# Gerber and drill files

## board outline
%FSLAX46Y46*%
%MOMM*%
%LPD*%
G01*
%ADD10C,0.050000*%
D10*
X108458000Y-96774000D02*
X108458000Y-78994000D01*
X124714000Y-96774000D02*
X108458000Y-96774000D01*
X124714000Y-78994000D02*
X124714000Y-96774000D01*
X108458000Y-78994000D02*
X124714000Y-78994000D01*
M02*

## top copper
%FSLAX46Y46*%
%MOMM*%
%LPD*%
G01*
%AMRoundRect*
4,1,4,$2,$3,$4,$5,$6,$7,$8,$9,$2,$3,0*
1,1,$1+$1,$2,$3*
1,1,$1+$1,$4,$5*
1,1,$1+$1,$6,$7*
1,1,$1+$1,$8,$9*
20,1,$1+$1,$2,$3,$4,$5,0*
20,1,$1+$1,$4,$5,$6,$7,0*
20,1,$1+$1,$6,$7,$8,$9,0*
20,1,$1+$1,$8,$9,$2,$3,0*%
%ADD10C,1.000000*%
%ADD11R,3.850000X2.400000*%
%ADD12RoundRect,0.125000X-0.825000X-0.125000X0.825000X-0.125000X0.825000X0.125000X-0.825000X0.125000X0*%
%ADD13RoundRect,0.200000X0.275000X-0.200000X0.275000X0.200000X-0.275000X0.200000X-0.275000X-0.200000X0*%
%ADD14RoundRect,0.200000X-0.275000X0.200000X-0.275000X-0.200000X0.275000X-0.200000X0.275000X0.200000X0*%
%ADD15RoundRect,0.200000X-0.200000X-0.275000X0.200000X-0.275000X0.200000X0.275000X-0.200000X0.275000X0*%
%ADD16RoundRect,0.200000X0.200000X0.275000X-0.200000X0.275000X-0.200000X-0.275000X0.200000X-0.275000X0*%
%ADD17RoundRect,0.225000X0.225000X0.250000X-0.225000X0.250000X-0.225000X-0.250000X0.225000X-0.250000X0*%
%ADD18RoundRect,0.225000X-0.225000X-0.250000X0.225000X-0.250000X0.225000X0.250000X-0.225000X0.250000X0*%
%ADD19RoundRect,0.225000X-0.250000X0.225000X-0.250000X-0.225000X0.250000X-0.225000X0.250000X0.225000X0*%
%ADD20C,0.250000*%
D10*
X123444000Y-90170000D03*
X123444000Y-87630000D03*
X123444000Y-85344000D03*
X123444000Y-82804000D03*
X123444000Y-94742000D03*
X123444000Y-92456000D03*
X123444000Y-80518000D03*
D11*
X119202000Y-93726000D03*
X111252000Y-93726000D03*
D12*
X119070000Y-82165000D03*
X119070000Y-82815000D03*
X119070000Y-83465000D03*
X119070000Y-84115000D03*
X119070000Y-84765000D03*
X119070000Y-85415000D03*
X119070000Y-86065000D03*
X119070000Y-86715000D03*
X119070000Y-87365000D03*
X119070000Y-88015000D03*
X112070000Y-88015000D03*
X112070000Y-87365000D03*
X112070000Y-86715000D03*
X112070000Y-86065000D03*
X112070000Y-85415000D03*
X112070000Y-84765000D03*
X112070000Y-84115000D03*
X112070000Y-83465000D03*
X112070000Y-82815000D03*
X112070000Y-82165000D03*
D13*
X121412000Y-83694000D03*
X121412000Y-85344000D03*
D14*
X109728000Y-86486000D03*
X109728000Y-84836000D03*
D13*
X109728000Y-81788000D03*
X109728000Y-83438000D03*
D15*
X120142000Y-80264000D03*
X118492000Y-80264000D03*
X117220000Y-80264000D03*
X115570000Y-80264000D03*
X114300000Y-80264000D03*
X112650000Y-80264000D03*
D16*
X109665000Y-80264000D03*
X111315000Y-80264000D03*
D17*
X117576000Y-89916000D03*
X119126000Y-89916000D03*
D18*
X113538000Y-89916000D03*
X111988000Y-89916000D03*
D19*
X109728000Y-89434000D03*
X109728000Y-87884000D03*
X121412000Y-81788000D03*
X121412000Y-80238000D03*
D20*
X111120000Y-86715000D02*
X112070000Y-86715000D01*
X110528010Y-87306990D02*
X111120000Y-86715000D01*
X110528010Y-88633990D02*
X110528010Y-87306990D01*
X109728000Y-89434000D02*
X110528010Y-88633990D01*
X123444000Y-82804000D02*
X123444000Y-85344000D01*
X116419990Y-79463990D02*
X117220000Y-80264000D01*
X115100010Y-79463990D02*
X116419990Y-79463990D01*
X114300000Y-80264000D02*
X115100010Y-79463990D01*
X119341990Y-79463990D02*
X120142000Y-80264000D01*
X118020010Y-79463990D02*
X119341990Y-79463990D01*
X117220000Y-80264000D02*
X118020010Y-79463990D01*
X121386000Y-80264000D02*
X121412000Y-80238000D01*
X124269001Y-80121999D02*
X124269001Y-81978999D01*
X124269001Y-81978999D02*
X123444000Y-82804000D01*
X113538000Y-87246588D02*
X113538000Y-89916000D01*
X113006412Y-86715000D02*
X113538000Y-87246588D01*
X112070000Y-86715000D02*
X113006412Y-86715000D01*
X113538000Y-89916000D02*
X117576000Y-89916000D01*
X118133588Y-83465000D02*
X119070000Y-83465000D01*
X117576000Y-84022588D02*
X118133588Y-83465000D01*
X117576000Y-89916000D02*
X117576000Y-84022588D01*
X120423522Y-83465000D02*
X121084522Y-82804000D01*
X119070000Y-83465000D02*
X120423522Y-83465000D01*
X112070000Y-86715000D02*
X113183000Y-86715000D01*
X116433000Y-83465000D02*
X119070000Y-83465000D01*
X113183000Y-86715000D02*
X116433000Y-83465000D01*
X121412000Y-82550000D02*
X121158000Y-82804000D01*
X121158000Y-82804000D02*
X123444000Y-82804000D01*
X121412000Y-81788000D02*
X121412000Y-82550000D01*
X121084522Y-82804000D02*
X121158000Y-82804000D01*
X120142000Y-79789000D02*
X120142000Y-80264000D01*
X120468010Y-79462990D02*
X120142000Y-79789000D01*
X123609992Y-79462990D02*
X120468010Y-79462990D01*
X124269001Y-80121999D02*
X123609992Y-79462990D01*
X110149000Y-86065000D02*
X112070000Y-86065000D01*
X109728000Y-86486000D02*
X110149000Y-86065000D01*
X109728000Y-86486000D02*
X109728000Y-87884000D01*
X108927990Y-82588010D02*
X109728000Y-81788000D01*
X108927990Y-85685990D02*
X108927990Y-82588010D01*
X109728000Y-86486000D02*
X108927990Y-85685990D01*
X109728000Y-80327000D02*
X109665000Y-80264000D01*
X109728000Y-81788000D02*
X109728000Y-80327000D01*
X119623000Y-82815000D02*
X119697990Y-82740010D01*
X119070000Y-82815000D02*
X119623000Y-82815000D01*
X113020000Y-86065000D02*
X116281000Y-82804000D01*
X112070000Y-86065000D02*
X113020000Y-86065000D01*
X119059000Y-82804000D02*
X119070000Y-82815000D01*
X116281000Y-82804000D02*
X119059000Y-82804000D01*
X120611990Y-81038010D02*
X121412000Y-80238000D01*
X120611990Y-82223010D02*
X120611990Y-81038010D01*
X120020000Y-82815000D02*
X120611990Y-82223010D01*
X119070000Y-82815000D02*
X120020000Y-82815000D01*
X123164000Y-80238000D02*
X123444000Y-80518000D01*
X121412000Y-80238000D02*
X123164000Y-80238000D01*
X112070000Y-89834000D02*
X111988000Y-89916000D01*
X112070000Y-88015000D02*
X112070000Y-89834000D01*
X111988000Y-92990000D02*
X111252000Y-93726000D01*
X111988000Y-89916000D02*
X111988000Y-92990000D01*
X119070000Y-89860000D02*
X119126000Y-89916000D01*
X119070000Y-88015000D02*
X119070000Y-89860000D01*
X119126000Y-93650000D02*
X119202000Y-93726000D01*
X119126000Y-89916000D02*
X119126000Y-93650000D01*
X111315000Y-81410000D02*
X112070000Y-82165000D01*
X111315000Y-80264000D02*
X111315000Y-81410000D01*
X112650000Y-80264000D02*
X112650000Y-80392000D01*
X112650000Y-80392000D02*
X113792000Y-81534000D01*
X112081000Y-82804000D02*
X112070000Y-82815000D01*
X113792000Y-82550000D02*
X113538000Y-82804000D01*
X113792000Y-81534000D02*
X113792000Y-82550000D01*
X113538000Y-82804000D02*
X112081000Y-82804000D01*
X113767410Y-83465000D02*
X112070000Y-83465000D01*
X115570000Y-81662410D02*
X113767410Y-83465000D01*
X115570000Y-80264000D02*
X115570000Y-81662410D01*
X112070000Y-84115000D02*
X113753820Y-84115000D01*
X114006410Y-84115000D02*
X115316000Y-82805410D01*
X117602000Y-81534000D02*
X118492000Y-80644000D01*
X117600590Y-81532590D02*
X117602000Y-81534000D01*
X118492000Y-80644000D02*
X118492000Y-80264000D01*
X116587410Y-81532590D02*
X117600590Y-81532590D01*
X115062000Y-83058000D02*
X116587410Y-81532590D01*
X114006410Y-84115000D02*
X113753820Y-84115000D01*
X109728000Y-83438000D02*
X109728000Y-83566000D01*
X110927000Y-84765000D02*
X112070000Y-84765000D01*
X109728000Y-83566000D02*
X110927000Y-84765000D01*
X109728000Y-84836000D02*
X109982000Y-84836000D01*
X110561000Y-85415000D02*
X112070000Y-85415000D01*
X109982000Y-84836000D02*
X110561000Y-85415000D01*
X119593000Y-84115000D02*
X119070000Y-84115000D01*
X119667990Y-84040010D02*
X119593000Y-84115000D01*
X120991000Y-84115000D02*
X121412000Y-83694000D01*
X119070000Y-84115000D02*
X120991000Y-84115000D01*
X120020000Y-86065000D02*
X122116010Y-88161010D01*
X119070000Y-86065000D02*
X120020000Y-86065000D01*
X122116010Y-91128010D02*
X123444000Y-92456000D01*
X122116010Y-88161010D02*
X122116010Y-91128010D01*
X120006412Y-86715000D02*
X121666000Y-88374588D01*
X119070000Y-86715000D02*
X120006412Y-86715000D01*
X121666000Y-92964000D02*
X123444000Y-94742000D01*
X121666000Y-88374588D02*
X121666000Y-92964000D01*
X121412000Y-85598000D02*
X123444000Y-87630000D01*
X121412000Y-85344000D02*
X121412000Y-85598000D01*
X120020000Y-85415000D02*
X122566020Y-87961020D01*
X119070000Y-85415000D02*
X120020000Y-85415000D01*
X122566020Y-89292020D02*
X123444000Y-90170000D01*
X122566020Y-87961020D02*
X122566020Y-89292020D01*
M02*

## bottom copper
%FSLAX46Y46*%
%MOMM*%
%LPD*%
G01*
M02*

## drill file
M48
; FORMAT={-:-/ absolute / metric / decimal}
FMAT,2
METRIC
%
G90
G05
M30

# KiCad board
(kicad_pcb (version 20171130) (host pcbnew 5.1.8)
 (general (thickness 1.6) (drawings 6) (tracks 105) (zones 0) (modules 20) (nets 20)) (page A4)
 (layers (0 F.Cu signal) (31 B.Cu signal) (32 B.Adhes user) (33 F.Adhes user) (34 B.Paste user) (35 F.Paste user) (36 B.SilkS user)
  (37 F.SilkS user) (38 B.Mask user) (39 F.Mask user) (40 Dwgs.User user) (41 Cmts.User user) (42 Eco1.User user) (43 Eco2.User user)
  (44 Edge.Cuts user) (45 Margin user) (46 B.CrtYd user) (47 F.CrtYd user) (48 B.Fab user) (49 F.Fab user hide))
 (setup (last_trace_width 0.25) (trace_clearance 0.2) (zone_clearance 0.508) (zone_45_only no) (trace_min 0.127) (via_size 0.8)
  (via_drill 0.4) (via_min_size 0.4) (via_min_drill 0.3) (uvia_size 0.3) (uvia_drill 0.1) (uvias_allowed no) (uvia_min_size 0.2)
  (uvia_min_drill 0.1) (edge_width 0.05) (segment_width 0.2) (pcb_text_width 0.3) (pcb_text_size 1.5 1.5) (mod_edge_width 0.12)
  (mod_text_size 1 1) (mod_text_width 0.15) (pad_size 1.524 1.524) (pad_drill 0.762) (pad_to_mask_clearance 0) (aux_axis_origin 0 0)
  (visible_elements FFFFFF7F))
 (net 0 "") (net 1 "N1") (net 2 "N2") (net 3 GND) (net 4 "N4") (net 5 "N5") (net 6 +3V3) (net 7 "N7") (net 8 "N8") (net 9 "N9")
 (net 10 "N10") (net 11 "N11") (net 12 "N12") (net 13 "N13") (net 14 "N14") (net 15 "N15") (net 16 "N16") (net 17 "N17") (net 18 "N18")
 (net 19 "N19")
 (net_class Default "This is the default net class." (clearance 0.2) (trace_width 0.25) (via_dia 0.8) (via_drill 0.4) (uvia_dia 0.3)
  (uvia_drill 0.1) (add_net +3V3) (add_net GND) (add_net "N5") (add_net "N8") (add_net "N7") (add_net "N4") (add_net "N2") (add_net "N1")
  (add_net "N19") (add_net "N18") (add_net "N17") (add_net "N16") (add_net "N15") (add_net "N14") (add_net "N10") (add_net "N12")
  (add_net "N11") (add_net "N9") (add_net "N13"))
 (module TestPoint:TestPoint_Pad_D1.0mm (layer F.Cu) (at 123.444 90.17)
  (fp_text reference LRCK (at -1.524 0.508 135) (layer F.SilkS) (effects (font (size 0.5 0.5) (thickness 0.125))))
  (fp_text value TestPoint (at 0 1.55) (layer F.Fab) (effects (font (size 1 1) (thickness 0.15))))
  (pad 1 smd circle (at 0 0) (size 1 1) (layers F.Cu F.Mask) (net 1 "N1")))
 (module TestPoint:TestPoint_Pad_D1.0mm (layer F.Cu) (at 123.444 87.63)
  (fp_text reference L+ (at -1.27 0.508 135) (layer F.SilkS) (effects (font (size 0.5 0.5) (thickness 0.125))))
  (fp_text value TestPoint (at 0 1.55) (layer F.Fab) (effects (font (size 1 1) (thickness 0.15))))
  (pad 1 smd circle (at 0 0) (size 1 1) (layers F.Cu F.Mask) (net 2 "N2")))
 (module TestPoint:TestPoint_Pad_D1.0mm (layer F.Cu) (at 123.444 85.344)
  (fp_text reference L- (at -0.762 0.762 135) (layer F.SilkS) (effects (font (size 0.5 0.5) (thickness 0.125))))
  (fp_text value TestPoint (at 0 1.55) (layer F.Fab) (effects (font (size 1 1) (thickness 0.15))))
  (pad 1 smd circle (at 0 0) (size 1 1) (layers F.Cu F.Mask) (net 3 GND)))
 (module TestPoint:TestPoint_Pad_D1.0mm (layer F.Cu) (at 123.444 82.804)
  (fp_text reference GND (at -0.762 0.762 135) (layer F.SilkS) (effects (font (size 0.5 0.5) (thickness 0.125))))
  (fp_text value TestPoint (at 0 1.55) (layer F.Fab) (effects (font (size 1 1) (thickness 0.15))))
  (pad 1 smd circle (at 0 0) (size 1 1) (layers F.Cu F.Mask) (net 3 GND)))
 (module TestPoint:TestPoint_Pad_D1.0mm (layer F.Cu) (at 123.444 94.742)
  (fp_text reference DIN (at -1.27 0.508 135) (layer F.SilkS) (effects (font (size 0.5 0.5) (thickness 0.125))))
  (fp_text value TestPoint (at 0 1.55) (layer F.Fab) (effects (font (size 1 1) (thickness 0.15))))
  (pad 1 smd circle (at 0 0) (size 1 1) (layers F.Cu F.Mask) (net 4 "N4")))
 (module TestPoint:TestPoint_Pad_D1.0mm (layer F.Cu) (at 123.444 92.456)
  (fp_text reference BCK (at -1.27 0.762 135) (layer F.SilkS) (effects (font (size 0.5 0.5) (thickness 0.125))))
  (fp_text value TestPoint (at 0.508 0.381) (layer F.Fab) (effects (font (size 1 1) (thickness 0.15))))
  (pad 1 smd circle (at 0 0) (size 1 1) (layers F.Cu F.Mask) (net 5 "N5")))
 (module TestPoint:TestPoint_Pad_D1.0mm (layer F.Cu) (at 123.444 80.518)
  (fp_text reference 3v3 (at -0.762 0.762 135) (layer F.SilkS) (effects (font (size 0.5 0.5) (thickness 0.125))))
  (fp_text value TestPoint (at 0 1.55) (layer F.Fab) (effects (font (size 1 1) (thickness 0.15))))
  (pad 1 smd circle (at 0 0) (size 1 1) (layers F.Cu F.Mask) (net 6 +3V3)))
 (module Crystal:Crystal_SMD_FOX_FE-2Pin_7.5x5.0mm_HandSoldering (layer F.Cu) (at 115.227 93.726)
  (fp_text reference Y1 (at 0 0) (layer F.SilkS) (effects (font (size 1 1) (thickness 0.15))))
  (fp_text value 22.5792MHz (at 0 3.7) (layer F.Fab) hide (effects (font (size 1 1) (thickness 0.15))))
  (pad 2 smd rect (at 3.975 0) (size 3.85 2.4) (layers F.Cu F.Paste F.Mask) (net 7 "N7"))
  (pad 1 smd rect (at -3.975 0) (size 3.85 2.4) (layers F.Cu F.Paste F.Mask) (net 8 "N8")))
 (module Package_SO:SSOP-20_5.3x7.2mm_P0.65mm (layer F.Cu) (at 115.57 85.09)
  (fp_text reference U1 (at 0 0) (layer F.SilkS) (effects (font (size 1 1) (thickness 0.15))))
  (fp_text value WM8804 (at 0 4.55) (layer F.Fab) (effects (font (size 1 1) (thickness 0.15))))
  (pad 20 smd roundrect (at 3.5 -2.925) (size 1.9 0.5) (layers F.Cu F.Paste F.Mask) (roundrect_rratio 0.25) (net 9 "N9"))
  (pad 19 smd roundrect (at 3.5 -2.275) (size 1.9 0.5) (layers F.Cu F.Paste F.Mask) (roundrect_rratio 0.25) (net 6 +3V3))
  (pad 18 smd roundrect (at 3.5 -1.625) (size 1.9 0.5) (layers F.Cu F.Paste F.Mask) (roundrect_rratio 0.25) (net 3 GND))
  (pad 17 smd roundrect (at 3.5 -0.975) (size 1.9 0.5) (layers F.Cu F.Paste F.Mask) (roundrect_rratio 0.25) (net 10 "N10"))
  (pad 16 smd roundrect (at 3.5 -0.325) (size 1.9 0.5) (layers F.Cu F.Paste F.Mask) (roundrect_rratio 0.25) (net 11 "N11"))
  (pad 15 smd roundrect (at 3.5 0.325) (size 1.9 0.5) (layers F.Cu F.Paste F.Mask) (roundrect_rratio 0.25) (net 1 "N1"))
  (pad 14 smd roundrect (at 3.5 0.975) (size 1.9 0.5) (layers F.Cu F.Paste F.Mask) (roundrect_rratio 0.25) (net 5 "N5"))
  (pad 13 smd roundrect (at 3.5 1.625) (size 1.9 0.5) (layers F.Cu F.Paste F.Mask) (roundrect_rratio 0.25) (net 4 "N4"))
  (pad 12 smd roundrect (at 3.5 2.275) (size 1.9 0.5) (layers F.Cu F.Paste F.Mask) (roundrect_rratio 0.25) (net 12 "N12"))
  (pad 11 smd roundrect (at 3.5 2.925) (size 1.9 0.5) (layers F.Cu F.Paste F.Mask) (roundrect_rratio 0.25) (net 7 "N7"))
  (pad 10 smd roundrect (at -3.5 2.925) (size 1.9 0.5) (layers F.Cu F.Paste F.Mask) (roundrect_rratio 0.25) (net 8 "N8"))
  (pad 9 smd roundrect (at -3.5 2.275) (size 1.9 0.5) (layers F.Cu F.Paste F.Mask) (roundrect_rratio 0.25) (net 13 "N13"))
  (pad 8 smd roundrect (at -3.5 1.625) (size 1.9 0.5) (layers F.Cu F.Paste F.Mask) (roundrect_rratio 0.25) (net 3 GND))
  (pad 7 smd roundrect (at -3.5 0.975) (size 1.9 0.5) (layers F.Cu F.Paste F.Mask) (roundrect_rratio 0.25) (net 6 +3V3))
  (pad 6 smd roundrect (at -3.5 0.325) (size 1.9 0.5) (layers F.Cu F.Paste F.Mask) (roundrect_rratio 0.25) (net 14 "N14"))
  (pad 5 smd roundrect (at -3.5 -0.325) (size 1.9 0.5) (layers F.Cu F.Paste F.Mask) (roundrect_rratio 0.25) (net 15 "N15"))
  (pad 4 smd roundrect (at -3.5 -0.975) (size 1.9 0.5) (layers F.Cu F.Paste F.Mask) (roundrect_rratio 0.25) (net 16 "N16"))
  (pad 3 smd roundrect (at -3.5 -1.625) (size 1.9 0.5) (layers F.Cu F.Paste F.Mask) (roundrect_rratio 0.25) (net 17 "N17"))
  (pad 2 smd roundrect (at -3.5 -2.275) (size 1.9 0.5) (layers F.Cu F.Paste F.Mask) (roundrect_rratio 0.25) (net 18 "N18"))
  (pad 1 smd roundrect (at -3.5 -2.925) (size 1.9 0.5) (layers F.Cu F.Paste F.Mask) (roundrect_rratio 0.25) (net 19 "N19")))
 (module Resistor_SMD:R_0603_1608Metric (layer F.Cu) (at 121.412 84.519 90)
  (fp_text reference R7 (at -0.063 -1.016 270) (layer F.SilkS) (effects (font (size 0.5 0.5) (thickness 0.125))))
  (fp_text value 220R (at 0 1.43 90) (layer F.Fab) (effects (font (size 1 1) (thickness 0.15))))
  (pad 2 smd roundrect (at 0.825 0 90) (size 0.8 0.95) (layers F.Cu F.Paste F.Mask) (roundrect_rratio 0.25) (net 10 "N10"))
  (pad 1 smd roundrect (at -0.825 0 90) (size 0.8 0.95) (layers F.Cu F.Paste F.Mask) (roundrect_rratio 0.25) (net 2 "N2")))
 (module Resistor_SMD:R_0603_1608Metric (layer F.Cu) (at 109.728 85.661 270)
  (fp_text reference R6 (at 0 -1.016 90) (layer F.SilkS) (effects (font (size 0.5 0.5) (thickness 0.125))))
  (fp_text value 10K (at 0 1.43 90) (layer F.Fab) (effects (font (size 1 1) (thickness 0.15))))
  (pad 2 smd roundrect (at 0.825 0 270) (size 0.8 0.95) (layers F.Cu F.Paste F.Mask) (roundrect_rratio 0.25) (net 6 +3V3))
  (pad 1 smd roundrect (at -0.825 0 270) (size 0.8 0.95) (layers F.Cu F.Paste F.Mask) (roundrect_rratio 0.25) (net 14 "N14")))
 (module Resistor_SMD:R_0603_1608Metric (layer F.Cu) (at 109.728 82.613 90)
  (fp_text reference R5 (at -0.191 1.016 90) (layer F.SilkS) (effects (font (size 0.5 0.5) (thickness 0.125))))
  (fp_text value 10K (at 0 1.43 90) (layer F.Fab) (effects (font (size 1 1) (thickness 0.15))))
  (pad 2 smd roundrect (at 0.825 0 90) (size 0.8 0.95) (layers F.Cu F.Paste F.Mask) (roundrect_rratio 0.25) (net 6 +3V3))
  (pad 1 smd roundrect (at -0.825 0 90) (size 0.8 0.95) (layers F.Cu F.Paste F.Mask) (roundrect_rratio 0.25) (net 15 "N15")))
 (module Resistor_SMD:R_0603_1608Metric (layer F.Cu) (at 119.317 80.264)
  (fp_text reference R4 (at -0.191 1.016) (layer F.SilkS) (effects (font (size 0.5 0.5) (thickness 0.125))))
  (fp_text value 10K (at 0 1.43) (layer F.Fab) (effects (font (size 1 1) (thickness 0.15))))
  (pad 2 smd roundrect (at 0.825 0) (size 0.8 0.95) (layers F.Cu F.Paste F.Mask) (roundrect_rratio 0.25) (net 3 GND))
  (pad 1 smd roundrect (at -0.825 0) (size 0.8 0.95) (layers F.Cu F.Paste F.Mask) (roundrect_rratio 0.25) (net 16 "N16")))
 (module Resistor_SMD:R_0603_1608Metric (layer F.Cu) (at 116.395 80.264)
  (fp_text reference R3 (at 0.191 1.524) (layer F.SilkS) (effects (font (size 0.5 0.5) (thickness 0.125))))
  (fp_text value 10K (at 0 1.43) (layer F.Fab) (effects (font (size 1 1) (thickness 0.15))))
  (pad 2 smd roundrect (at 0.825 0) (size 0.8 0.95) (layers F.Cu F.Paste F.Mask) (roundrect_rratio 0.25) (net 3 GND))
  (pad 1 smd roundrect (at -0.825 0) (size 0.8 0.95) (layers F.Cu F.Paste F.Mask) (roundrect_rratio 0.25) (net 17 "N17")))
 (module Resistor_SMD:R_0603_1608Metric (layer F.Cu) (at 113.475 80.264)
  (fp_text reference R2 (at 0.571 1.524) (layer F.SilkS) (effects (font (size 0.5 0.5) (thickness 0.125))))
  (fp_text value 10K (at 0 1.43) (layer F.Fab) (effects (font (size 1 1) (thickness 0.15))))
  (pad 2 smd roundrect (at 0.825 0) (size 0.8 0.95) (layers F.Cu F.Paste F.Mask) (roundrect_rratio 0.25) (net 3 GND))
  (pad 1 smd roundrect (at -0.825 0) (size 0.8 0.95) (layers F.Cu F.Paste F.Mask) (roundrect_rratio 0.25) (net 18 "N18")))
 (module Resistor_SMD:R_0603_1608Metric (layer F.Cu) (at 110.49 80.264 180)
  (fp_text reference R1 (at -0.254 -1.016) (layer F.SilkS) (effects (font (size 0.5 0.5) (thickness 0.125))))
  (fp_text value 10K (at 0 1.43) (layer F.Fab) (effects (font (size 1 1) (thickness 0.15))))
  (pad 2 smd roundrect (at 0.825 0 180) (size 0.8 0.95) (layers F.Cu F.Paste F.Mask) (roundrect_rratio 0.25) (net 6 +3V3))
  (pad 1 smd roundrect (at -0.825 0 180) (size 0.8 0.95) (layers F.Cu F.Paste F.Mask) (roundrect_rratio 0.25) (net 19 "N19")))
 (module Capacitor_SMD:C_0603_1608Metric (layer F.Cu) (at 118.351 89.916 180)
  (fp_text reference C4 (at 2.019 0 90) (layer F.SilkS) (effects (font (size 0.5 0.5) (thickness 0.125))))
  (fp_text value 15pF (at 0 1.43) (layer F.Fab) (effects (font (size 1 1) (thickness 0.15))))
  (pad 2 smd roundrect (at 0.775 0 180) (size 0.9 0.95) (layers F.Cu F.Paste F.Mask) (roundrect_rratio 0.25) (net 3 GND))
  (pad 1 smd roundrect (at -0.775 0 180) (size 0.9 0.95) (layers F.Cu F.Paste F.Mask) (roundrect_rratio 0.25) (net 7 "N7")))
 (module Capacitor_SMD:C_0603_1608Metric (layer F.Cu) (at 112.763 89.916)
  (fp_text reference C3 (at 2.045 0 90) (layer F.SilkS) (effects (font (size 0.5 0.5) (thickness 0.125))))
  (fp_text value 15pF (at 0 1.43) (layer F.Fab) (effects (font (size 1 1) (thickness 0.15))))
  (pad 2 smd roundrect (at 0.775 0) (size 0.9 0.95) (layers F.Cu F.Paste F.Mask) (roundrect_rratio 0.25) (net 3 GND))
  (pad 1 smd roundrect (at -0.775 0) (size 0.9 0.95) (layers F.Cu F.Paste F.Mask) (roundrect_rratio 0.25) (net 8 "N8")))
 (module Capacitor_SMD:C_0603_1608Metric (layer F.Cu) (at 109.728 88.659 270)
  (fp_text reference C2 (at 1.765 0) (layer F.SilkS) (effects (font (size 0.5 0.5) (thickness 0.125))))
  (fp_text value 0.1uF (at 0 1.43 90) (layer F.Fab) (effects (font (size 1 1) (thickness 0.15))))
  (pad 2 smd roundrect (at 0.775 0 270) (size 0.9 0.95) (layers F.Cu F.Paste F.Mask) (roundrect_rratio 0.25) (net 3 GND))
  (pad 1 smd roundrect (at -0.775 0 270) (size 0.9 0.95) (layers F.Cu F.Paste F.Mask) (roundrect_rratio 0.25) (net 6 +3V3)))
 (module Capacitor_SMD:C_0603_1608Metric (layer F.Cu) (at 121.412 81.013 270)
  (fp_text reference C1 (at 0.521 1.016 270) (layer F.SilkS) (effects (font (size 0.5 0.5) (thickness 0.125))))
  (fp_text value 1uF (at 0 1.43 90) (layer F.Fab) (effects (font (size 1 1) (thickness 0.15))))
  (pad 2 smd roundrect (at 0.775 0 270) (size 0.9 0.95) (layers F.Cu F.Paste F.Mask) (roundrect_rratio 0.25) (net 3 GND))
  (pad 1 smd roundrect (at -0.775 0 270) (size 0.9 0.95) (layers F.Cu F.Paste F.Mask) (roundrect_rratio 0.25) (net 6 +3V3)))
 (gr_line (start 108.458 96.774) (end 108.458 78.994) (layer Edge.Cuts) (width 0.05))
 (gr_line (start 124.714 96.774) (end 108.458 96.774) (layer Edge.Cuts) (width 0.05))
 (gr_line (start 124.714 78.994) (end 124.714 96.774) (layer Edge.Cuts) (width 0.05))
 (gr_line (start 108.458 78.994) (end 124.714 78.994) (layer Edge.Cuts) (width 0.05))
 (segment (start 111.12 86.715) (end 112.07 86.715) (width 0.25) (layer F.Cu) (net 3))
 (segment (start 110.52801 87.30699) (end 111.12 86.715) (width 0.25) (layer F.Cu) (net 3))
 (segment (start 110.52801 88.63399) (end 110.52801 87.30699) (width 0.25) (layer F.Cu) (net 3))
 (segment (start 109.728 89.434) (end 110.52801 88.63399) (width 0.25) (layer F.Cu) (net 3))
 (segment (start 123.444 82.804) (end 123.444 85.344) (width 0.25) (layer F.Cu) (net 3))
 (segment (start 116.41999 79.46399) (end 117.22 80.264) (width 0.25) (layer F.Cu) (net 3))
 (segment (start 115.10001 79.46399) (end 116.41999 79.46399) (width 0.25) (layer F.Cu) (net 3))
 (segment (start 114.3 80.264) (end 115.10001 79.46399) (width 0.25) (layer F.Cu) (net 3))
 (segment (start 119.34199 79.46399) (end 120.142 80.264) (width 0.25) (layer F.Cu) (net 3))
 (segment (start 118.02001 79.46399) (end 119.34199 79.46399) (width 0.25) (layer F.Cu) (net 3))
 (segment (start 117.22 80.264) (end 118.02001 79.46399) (width 0.25) (layer F.Cu) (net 3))
 (segment (start 121.386 80.264) (end 121.412 80.238) (width 0.25) (layer F.Cu) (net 6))
 (segment (start 124.269001 80.121999) (end 124.269001 81.978999) (width 0.25) (layer F.Cu) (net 3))
 (segment (start 124.269001 81.978999) (end 123.444 82.804) (width 0.25) (layer F.Cu) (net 3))
 (segment (start 113.538 87.246588) (end 113.538 89.916) (width 0.25) (layer F.Cu) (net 3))
 (segment (start 113.006412 86.715) (end 113.538 87.246588) (width 0.25) (layer F.Cu) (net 3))
 (segment (start 112.07 86.715) (end 113.006412 86.715) (width 0.25) (layer F.Cu) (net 3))
 (segment (start 113.538 89.916) (end 117.576 89.916) (width 0.25) (layer F.Cu) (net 3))
 (segment (start 118.133588 83.465) (end 119.07 83.465) (width 0.25) (layer F.Cu) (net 3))
 (segment (start 117.576 84.022588) (end 118.133588 83.465) (width 0.25) (layer F.Cu) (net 3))
 (segment (start 117.576 89.916) (end 117.576 84.022588) (width 0.25) (layer F.Cu) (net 3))
 (segment (start 120.423522 83.465) (end 121.084522 82.804) (width 0.25) (layer F.Cu) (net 3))
 (segment (start 119.07 83.465) (end 120.423522 83.465) (width 0.25) (layer F.Cu) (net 3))
 (segment (start 112.07 86.715) (end 113.183 86.715) (width 0.25) (layer F.Cu) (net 3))
 (segment (start 116.433 83.465) (end 119.07 83.465) (width 0.25) (layer F.Cu) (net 3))
 (segment (start 113.183 86.715) (end 116.433 83.465) (width 0.25) (layer F.Cu) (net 3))
 (segment (start 121.412 82.55) (end 121.158 82.804) (width 0.25) (layer F.Cu) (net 3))
 (segment (start 121.158 82.804) (end 123.444 82.804) (width 0.25) (layer F.Cu) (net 3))
 (segment (start 121.412 81.788) (end 121.412 82.55) (width 0.25) (layer F.Cu) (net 3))
 (segment (start 121.084522 82.804) (end 121.158 82.804) (width 0.25) (layer F.Cu) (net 3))
 (segment (start 120.142 79.789) (end 120.142 80.264) (width 0.25) (layer F.Cu) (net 3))
 (segment (start 120.46801 79.46299) (end 120.142 79.789) (width 0.25) (layer F.Cu) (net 3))
 (segment (start 123.609992 79.46299) (end 120.46801 79.46299) (width 0.25) (layer F.Cu) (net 3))
 (segment (start 124.269001 80.121999) (end 123.609992 79.46299) (width 0.25) (layer F.Cu) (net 3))
 (segment (start 110.149 86.065) (end 112.07 86.065) (width 0.25) (layer F.Cu) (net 6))
 (segment (start 109.728 86.486) (end 110.149 86.065) (width 0.25) (layer F.Cu) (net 6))
 (segment (start 109.728 86.486) (end 109.728 87.884) (width 0.25) (layer F.Cu) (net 6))
 (segment (start 108.92799 82.58801) (end 109.728 81.788) (width 0.25) (layer F.Cu) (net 6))
 (segment (start 108.92799 85.68599) (end 108.92799 82.58801) (width 0.25) (layer F.Cu) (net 6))
 (segment (start 109.728 86.486) (end 108.92799 85.68599) (width 0.25) (layer F.Cu) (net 6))
 (segment (start 109.728 80.327) (end 109.665 80.264) (width 0.25) (layer F.Cu) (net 6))
 (segment (start 109.728 81.788) (end 109.728 80.327) (width 0.25) (layer F.Cu) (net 6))
 (segment (start 119.623 82.815) (end 119.69799 82.74001) (width 0.25) (layer F.Cu) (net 6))
 (segment (start 119.07 82.815) (end 119.623 82.815) (width 0.25) (layer F.Cu) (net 6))
 (segment (start 113.02 86.065) (end 116.281 82.804) (width 0.25) (layer F.Cu) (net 6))
 (segment (start 112.07 86.065) (end 113.02 86.065) (width 0.25) (layer F.Cu) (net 6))
 (segment (start 119.059 82.804) (end 119.07 82.815) (width 0.25) (layer F.Cu) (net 6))
 (segment (start 116.281 82.804) (end 119.059 82.804) (width 0.25) (layer F.Cu) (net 6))
 (segment (start 120.61199 81.03801) (end 121.412 80.238) (width 0.25) (layer F.Cu) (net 6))
 (segment (start 120.61199 82.22301) (end 120.61199 81.03801) (width 0.25) (layer F.Cu) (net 6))
 (segment (start 120.02 82.815) (end 120.61199 82.22301) (width 0.25) (layer F.Cu) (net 6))
 (segment (start 119.07 82.815) (end 120.02 82.815) (width 0.25) (layer F.Cu) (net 6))
 (segment (start 123.164 80.238) (end 123.444 80.518) (width 0.25) (layer F.Cu) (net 6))
 (segment (start 121.412 80.238) (end 123.164 80.238) (width 0.25) (layer F.Cu) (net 6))
 (segment (start 112.07 89.834) (end 111.988 89.916) (width 0.25) (layer F.Cu) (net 8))
 (segment (start 112.07 88.015) (end 112.07 89.834) (width 0.25) (layer F.Cu) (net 8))
 (segment (start 111.988 92.99) (end 111.252 93.726) (width 0.25) (layer F.Cu) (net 8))
 (segment (start 111.988 89.916) (end 111.988 92.99) (width 0.25) (layer F.Cu) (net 8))
 (segment (start 119.07 89.86) (end 119.126 89.916) (width 0.25) (layer F.Cu) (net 7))
 (segment (start 119.07 88.015) (end 119.07 89.86) (width 0.25) (layer F.Cu) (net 7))
 (segment (start 119.126 93.65) (end 119.202 93.726) (width 0.25) (layer F.Cu) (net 7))
 (segment (start 119.126 89.916) (end 119.126 93.65) (width 0.25) (layer F.Cu) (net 7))
 (segment (start 111.315 81.41) (end 112.07 82.165) (width 0.25) (layer F.Cu) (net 19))
 (segment (start 111.315 80.264) (end 111.315 81.41) (width 0.25) (layer F.Cu) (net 19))
 (segment (start 112.65 80.264) (end 112.65 80.392) (width 0.25) (layer F.Cu) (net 18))
 (segment (start 112.65 80.392) (end 113.792 81.534) (width 0.25) (layer F.Cu) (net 18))
 (segment (start 112.081 82.804) (end 112.07 82.815) (width 0.25) (layer F.Cu) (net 18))
 (segment (start 113.792 82.55) (end 113.538 82.804) (width 0.25) (layer F.Cu) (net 18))
 (segment (start 113.792 81.534) (end 113.792 82.55) (width 0.25) (layer F.Cu) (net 18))
 (segment (start 113.538 82.804) (end 112.081 82.804) (width 0.25) (layer F.Cu) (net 18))
 (segment (start 113.76741 83.465) (end 112.07 83.465) (width 0.25) (layer F.Cu) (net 17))
 (segment (start 115.57 81.66241) (end 113.76741 83.465) (width 0.25) (layer F.Cu) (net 17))
 (segment (start 115.57 80.264) (end 115.57 81.66241) (width 0.25) (layer F.Cu) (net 17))
 (segment (start 112.07 84.115) (end 113.75382 84.115) (width 0.25) (layer F.Cu) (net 16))
 (segment (start 114.00641 84.115) (end 115.316 82.80541) (width 0.25) (layer F.Cu) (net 16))
 (segment (start 117.602 81.534) (end 118.492 80.644) (width 0.25) (layer F.Cu) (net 16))
 (segment (start 117.60059 81.53259) (end 117.602 81.534) (width 0.25) (layer F.Cu) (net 16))
 (segment (start 118.492 80.644) (end 118.492 80.264) (width 0.25) (layer F.Cu) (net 16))
 (segment (start 116.58741 81.53259) (end 117.60059 81.53259) (width 0.25) (layer F.Cu) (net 16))
 (segment (start 115.062 83.058) (end 116.58741 81.53259) (width 0.25) (layer F.Cu) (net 16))
 (segment (start 114.00641 84.115) (end 113.75382 84.115) (width 0.25) (layer F.Cu) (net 16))
 (segment (start 109.728 83.438) (end 109.728 83.566) (width 0.25) (layer F.Cu) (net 15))
 (segment (start 110.927 84.765) (end 112.07 84.765) (width 0.25) (layer F.Cu) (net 15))
 (segment (start 109.728 83.566) (end 110.927 84.765) (width 0.25) (layer F.Cu) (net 15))
 (segment (start 109.728 84.836) (end 109.982 84.836) (width 0.25) (layer F.Cu) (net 14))
 (segment (start 110.561 85.415) (end 112.07 85.415) (width 0.25) (layer F.Cu) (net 14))
 (segment (start 109.982 84.836) (end 110.561 85.415) (width 0.25) (layer F.Cu) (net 14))
 (segment (start 119.593 84.115) (end 119.07 84.115) (width 0.25) (layer F.Cu) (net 10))
 (segment (start 119.66799 84.04001) (end 119.593 84.115) (width 0.25) (layer F.Cu) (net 10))
 (segment (start 120.991 84.115) (end 121.412 83.694) (width 0.25) (layer F.Cu) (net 10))
 (segment (start 119.07 84.115) (end 120.991 84.115) (width 0.25) (layer F.Cu) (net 10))
 (segment (start 120.02 86.065) (end 122.11601 88.16101) (width 0.25) (layer F.Cu) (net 5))
 (segment (start 119.07 86.065) (end 120.02 86.065) (width 0.25) (layer F.Cu) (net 5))
 (segment (start 122.11601 91.12801) (end 123.444 92.456) (width 0.25) (layer F.Cu) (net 5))
 (segment (start 122.11601 88.16101) (end 122.11601 91.12801) (width 0.25) (layer F.Cu) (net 5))
 (segment (start 120.006412 86.715) (end 121.666 88.374588) (width 0.25) (layer F.Cu) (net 4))
 (segment (start 119.07 86.715) (end 120.006412 86.715) (width 0.25) (layer F.Cu) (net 4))
 (segment (start 121.666 92.964) (end 123.444 94.742) (width 0.25) (layer F.Cu) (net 4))
 (segment (start 121.666 88.374588) (end 121.666 92.964) (width 0.25) (layer F.Cu) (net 4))
 (segment (start 121.412 85.598) (end 123.444 87.63) (width 0.25) (layer F.Cu) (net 2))
 (segment (start 121.412 85.344) (end 121.412 85.598) (width 0.25) (layer F.Cu) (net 2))
 (segment (start 120.02 85.415) (end 122.56602 87.96102) (width 0.25) (layer F.Cu) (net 1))
 (segment (start 119.07 85.415) (end 120.02 85.415) (width 0.25) (layer F.Cu) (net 1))
 (segment (start 122.56602 89.29202) (end 123.444 90.17) (width 0.25) (layer F.Cu) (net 1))
 (segment (start 122.56602 87.96102) (end 122.56602 89.29202) (width 0.25) (layer F.Cu) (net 1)))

